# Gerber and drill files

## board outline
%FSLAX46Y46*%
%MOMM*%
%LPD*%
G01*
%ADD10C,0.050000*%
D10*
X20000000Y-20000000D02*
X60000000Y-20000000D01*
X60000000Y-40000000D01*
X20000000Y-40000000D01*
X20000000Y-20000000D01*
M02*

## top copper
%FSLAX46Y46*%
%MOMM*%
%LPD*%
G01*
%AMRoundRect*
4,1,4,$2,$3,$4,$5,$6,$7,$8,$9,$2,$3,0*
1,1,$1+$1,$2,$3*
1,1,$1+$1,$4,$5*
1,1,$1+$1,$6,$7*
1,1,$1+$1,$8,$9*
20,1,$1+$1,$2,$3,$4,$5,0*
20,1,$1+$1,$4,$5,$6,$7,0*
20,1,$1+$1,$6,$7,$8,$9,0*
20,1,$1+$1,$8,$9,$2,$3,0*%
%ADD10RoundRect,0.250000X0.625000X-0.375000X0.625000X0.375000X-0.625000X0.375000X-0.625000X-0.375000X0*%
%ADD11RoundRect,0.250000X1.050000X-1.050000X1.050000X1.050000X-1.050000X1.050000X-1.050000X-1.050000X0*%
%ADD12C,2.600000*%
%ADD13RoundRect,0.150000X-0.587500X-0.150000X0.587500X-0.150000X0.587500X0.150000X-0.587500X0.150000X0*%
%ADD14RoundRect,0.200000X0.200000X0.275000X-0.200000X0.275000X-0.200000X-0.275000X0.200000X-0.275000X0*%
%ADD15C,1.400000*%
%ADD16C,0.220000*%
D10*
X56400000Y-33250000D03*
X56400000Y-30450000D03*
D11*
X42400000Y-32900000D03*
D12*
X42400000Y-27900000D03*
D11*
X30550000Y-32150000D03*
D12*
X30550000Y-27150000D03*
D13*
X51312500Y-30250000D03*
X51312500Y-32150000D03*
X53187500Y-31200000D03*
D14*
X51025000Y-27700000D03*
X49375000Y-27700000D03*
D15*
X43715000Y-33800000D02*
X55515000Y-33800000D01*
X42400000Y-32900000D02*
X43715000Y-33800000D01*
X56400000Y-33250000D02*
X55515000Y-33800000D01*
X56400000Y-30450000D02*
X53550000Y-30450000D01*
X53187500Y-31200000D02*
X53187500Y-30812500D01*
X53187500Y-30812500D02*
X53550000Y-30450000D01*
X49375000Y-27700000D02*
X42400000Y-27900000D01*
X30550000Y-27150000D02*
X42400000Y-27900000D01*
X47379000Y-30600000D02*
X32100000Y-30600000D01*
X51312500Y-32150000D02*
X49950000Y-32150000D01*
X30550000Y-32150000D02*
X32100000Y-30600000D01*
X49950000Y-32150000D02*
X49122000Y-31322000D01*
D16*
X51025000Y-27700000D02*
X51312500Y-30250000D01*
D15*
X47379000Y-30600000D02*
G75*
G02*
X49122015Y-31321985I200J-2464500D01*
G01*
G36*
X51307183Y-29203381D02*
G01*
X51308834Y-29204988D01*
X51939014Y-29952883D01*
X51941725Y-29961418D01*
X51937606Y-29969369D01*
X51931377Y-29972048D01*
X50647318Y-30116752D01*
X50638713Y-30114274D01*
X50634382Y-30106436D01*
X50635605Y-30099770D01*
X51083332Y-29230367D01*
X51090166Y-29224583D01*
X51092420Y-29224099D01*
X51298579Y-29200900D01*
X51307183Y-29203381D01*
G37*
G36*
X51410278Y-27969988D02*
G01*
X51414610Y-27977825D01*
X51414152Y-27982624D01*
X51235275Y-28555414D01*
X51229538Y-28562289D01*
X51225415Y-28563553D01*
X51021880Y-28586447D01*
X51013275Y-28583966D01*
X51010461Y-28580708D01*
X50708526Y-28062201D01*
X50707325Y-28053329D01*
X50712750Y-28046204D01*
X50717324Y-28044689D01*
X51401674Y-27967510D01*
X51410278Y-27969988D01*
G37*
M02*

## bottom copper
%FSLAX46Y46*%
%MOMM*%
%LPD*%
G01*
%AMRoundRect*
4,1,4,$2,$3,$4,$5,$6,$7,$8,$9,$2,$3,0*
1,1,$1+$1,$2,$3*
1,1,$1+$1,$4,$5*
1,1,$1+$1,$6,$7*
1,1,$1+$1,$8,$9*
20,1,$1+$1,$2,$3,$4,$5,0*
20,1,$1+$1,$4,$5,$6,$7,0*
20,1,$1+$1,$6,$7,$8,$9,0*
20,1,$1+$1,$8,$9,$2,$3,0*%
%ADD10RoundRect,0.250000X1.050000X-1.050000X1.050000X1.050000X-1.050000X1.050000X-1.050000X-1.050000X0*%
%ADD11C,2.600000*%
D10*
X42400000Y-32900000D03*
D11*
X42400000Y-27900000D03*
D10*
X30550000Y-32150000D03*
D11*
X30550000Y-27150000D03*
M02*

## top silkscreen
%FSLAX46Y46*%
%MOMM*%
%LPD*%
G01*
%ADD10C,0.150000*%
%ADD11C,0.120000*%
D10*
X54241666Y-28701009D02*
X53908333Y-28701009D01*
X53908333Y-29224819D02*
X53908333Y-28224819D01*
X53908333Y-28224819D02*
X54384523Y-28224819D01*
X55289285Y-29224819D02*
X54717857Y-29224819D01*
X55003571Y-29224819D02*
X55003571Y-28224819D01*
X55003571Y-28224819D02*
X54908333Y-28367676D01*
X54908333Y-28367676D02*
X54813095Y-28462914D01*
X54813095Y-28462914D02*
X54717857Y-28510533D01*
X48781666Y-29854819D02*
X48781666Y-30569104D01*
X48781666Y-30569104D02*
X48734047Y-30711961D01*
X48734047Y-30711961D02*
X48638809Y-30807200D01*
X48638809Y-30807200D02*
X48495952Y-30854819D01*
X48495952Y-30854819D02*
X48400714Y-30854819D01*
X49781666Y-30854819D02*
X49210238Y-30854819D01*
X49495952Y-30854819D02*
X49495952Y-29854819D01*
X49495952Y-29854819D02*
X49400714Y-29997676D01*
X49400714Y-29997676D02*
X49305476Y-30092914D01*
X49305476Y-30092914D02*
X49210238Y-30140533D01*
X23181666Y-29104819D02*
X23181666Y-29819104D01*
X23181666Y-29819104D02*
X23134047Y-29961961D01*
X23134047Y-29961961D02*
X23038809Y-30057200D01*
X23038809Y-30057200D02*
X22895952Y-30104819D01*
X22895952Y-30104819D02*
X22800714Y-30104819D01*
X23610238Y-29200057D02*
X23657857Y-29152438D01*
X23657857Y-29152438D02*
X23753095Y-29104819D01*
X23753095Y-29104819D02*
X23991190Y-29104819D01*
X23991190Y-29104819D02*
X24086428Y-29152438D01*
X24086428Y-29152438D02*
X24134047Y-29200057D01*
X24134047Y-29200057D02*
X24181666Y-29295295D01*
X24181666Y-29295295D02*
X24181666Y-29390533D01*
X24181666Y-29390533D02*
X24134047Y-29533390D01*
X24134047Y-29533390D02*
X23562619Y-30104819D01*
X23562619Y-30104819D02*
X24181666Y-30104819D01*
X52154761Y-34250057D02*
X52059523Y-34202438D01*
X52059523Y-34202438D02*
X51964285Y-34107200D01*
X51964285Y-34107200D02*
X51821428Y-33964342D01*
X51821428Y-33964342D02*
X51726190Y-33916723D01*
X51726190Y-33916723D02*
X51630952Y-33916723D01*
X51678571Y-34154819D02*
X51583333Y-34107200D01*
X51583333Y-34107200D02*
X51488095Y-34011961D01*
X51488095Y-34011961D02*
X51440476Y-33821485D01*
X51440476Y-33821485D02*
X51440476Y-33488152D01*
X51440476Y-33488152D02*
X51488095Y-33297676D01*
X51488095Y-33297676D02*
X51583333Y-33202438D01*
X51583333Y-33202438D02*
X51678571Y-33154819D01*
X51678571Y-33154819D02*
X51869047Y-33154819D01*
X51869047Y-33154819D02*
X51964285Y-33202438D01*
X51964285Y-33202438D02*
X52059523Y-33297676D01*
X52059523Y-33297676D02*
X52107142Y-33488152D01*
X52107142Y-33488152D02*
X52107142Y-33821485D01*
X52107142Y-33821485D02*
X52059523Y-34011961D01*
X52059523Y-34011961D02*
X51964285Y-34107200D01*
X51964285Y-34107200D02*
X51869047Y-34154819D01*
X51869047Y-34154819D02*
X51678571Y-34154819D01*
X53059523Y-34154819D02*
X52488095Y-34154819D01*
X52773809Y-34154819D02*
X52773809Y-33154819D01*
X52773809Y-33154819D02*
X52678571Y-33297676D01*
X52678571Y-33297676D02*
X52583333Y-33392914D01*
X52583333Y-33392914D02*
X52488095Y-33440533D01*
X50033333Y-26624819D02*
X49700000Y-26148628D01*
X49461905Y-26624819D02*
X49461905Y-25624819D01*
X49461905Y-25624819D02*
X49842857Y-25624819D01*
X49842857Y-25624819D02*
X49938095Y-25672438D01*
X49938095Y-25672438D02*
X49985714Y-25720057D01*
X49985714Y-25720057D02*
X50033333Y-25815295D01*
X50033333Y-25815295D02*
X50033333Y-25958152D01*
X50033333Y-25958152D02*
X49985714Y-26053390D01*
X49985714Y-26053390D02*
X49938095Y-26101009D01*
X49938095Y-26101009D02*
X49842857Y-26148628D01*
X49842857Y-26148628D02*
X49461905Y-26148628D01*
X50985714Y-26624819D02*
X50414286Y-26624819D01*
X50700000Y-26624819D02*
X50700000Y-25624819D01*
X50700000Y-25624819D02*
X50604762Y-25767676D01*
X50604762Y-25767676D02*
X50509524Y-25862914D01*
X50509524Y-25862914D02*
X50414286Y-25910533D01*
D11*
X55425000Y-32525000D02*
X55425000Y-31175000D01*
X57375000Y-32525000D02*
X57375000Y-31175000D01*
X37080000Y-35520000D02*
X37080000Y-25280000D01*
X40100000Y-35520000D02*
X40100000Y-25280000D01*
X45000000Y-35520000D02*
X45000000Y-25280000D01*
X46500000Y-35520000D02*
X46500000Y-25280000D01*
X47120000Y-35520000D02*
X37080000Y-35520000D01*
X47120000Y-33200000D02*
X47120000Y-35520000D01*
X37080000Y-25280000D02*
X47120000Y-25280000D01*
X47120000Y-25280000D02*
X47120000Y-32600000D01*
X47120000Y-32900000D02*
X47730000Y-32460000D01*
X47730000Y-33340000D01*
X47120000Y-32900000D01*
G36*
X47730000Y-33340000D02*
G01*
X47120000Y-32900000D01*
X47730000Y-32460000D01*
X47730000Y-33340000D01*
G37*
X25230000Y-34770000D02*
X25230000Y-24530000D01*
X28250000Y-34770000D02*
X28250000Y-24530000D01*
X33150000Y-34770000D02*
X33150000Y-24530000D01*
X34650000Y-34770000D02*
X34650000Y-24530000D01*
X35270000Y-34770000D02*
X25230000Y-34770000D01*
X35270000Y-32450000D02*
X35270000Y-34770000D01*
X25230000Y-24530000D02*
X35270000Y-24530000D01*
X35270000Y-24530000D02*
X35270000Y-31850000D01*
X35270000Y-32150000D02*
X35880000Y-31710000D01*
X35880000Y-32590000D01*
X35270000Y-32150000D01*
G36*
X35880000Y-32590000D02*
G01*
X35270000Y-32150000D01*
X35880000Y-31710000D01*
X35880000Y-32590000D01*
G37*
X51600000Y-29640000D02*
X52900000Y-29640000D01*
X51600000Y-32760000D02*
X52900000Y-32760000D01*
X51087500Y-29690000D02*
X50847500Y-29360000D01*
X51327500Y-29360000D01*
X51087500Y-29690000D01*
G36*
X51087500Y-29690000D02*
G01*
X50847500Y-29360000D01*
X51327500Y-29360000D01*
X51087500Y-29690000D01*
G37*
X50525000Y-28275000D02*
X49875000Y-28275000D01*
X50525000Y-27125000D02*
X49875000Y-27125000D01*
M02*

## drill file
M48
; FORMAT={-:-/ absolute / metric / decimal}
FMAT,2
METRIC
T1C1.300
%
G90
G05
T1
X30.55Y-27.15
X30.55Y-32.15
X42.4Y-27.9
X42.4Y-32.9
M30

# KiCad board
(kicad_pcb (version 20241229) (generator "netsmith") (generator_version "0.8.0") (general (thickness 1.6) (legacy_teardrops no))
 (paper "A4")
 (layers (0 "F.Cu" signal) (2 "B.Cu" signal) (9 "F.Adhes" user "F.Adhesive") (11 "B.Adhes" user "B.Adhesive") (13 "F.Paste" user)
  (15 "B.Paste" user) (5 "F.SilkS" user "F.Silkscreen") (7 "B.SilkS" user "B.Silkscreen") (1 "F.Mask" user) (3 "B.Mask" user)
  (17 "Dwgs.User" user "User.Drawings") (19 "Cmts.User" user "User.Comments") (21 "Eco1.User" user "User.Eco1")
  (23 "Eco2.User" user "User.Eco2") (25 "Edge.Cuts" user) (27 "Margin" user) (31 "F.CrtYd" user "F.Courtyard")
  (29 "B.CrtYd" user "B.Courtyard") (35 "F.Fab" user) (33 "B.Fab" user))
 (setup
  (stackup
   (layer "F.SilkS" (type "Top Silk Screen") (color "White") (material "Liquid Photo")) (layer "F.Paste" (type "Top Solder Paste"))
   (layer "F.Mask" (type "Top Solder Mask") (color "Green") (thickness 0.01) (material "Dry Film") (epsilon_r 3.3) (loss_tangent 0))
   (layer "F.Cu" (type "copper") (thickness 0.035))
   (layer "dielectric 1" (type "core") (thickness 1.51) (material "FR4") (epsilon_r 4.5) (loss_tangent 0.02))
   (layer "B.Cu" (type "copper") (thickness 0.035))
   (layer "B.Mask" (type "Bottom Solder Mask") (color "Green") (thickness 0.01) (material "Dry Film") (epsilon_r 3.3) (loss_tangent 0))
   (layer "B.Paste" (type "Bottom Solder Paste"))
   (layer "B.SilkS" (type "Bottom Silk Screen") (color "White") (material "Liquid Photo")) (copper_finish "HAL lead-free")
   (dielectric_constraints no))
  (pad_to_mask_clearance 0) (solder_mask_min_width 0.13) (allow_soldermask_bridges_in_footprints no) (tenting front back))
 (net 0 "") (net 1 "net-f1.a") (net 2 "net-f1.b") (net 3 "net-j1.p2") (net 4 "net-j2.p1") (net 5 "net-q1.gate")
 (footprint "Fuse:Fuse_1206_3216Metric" (layer "F.Cu") (at 56.4 31.85 90)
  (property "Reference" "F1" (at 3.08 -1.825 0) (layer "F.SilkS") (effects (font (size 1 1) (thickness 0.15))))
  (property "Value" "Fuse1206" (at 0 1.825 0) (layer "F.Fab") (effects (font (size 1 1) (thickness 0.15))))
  (pad "1" smd roundrect (at -1.4 0 90) (size 1.25 1.75) (layers "F.Cu" "F.Mask" "F.Paste") (roundrect_rratio 0.2) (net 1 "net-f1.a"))
  (pad "2" smd roundrect (at 1.4 0 90) (size 1.25 1.75) (layers "F.Cu" "F.Mask" "F.Paste") (roundrect_rratio 0.2) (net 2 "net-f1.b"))
  (fp_line (start -0.675 -0.975) (end 0.675 -0.975) (stroke (width 0.12) (type solid)) (layer "F.SilkS"))
  (fp_line (start -0.675 0.975) (end 0.675 0.975) (stroke (width 0.12) (type solid)) (layer "F.SilkS")))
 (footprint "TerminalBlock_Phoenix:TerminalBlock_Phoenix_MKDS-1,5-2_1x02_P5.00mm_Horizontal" (layer "F.Cu") (at 42.4 32.9 90)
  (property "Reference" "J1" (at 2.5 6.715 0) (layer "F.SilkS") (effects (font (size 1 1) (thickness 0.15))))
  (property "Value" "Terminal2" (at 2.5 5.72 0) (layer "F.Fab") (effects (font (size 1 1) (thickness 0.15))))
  (fp_line (start -2.62 -5.32) (end 7.62 -5.32) (stroke (width 0.12) (type solid)) (layer "F.SilkS"))
  (fp_line (start -2.62 -2.3) (end 7.62 -2.3) (stroke (width 0.12) (type solid)) (layer "F.SilkS"))
  (fp_line (start -2.62 2.6) (end 7.62 2.6) (stroke (width 0.12) (type solid)) (layer "F.SilkS"))
  (fp_line (start -2.62 4.1) (end 7.62 4.1) (stroke (width 0.12) (type solid)) (layer "F.SilkS"))
  (fp_line (start -2.62 4.72) (end -2.62 -5.32) (stroke (width 0.12) (type solid)) (layer "F.SilkS"))
  (fp_line (start -0.3 4.72) (end -2.62 4.72) (stroke (width 0.12) (type solid)) (layer "F.SilkS"))
  (fp_line (start 7.62 -5.32) (end 7.62 4.72) (stroke (width 0.12) (type solid)) (layer "F.SilkS"))
  (fp_line (start 7.62 4.72) (end 0.3 4.72) (stroke (width 0.12) (type solid)) (layer "F.SilkS"))
  (fp_poly (pts (xy 0 4.72) (xy 0.44 5.33) (xy -0.44 5.33)) (stroke (width 0.12) (type solid)) (fill yes) (layer "F.SilkS"))
  (pad "1" thru_hole roundrect (at 0 0 90) (size 2.6 2.6) (drill 1.3) (layers "*.Cu" "*.Mask") (remove_unused_layers no)
   (roundrect_rratio 0.096154) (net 1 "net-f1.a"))
  (pad "2" thru_hole circle (at 5 0 90) (size 2.6 2.6) (drill 1.3) (layers "*.Cu" "*.Mask") (remove_unused_layers no) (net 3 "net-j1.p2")))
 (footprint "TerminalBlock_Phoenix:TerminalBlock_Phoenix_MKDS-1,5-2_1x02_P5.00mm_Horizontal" (layer "F.Cu") (at 30.55 32.15 90)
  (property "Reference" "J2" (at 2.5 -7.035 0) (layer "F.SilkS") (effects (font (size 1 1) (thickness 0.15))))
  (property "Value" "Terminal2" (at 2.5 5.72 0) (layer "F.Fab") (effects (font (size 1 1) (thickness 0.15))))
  (fp_line (start -2.62 -5.32) (end 7.62 -5.32) (stroke (width 0.12) (type solid)) (layer "F.SilkS"))
  (fp_line (start -2.62 -2.3) (end 7.62 -2.3) (stroke (width 0.12) (type solid)) (layer "F.SilkS"))
  (fp_line (start -2.62 2.6) (end 7.62 2.6) (stroke (width 0.12) (type solid)) (layer "F.SilkS"))
  (fp_line (start -2.62 4.1) (end 7.62 4.1) (stroke (width 0.12) (type solid)) (layer "F.SilkS"))
  (fp_line (start -2.62 4.72) (end -2.62 -5.32) (stroke (width 0.12) (type solid)) (layer "F.SilkS"))
  (fp_line (start -0.3 4.72) (end -2.62 4.72) (stroke (width 0.12) (type solid)) (layer "F.SilkS"))
  (fp_line (start 7.62 -5.32) (end 7.62 4.72) (stroke (width 0.12) (type solid)) (layer "F.SilkS"))
  (fp_line (start 7.62 4.72) (end 0.3 4.72) (stroke (width 0.12) (type solid)) (layer "F.SilkS"))
  (fp_poly (pts (xy 0 4.72) (xy 0.44 5.33) (xy -0.44 5.33)) (stroke (width 0.12) (type solid)) (fill yes) (layer "F.SilkS"))
  (pad "1" thru_hole roundrect (at 0 0 90) (size 2.6 2.6) (drill 1.3) (layers "*.Cu" "*.Mask") (remove_unused_layers no)
   (roundrect_rratio 0.096154) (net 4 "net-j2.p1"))
  (pad "2" thru_hole circle (at 5 0 90) (size 2.6 2.6) (drill 1.3) (layers "*.Cu" "*.Mask") (remove_unused_layers no) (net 3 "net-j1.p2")))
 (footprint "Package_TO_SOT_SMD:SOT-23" (layer "F.Cu") (at 52.25 31.2)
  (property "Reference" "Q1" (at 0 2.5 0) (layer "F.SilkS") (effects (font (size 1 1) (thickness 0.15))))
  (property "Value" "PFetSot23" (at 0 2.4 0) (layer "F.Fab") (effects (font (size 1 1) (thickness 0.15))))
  (pad "1" smd roundrect (at -0.9375 -0.95) (size 1.475 0.6) (layers "F.Cu" "F.Mask" "F.Paste") (roundrect_rratio 0.25)
   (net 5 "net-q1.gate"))
  (pad "2" smd roundrect (at -0.9375 0.95) (size 1.475 0.6) (layers "F.Cu" "F.Mask" "F.Paste") (roundrect_rratio 0.25) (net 4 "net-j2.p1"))
  (pad "3" smd roundrect (at 0.9375 0) (size 1.475 0.6) (layers "F.Cu" "F.Mask" "F.Paste") (roundrect_rratio 0.25) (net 2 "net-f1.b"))
  (fp_line (start -0.65 -1.56) (end 0.65 -1.56) (stroke (width 0.12) (type solid)) (layer "F.SilkS"))
  (fp_line (start -0.65 1.56) (end 0.65 1.56) (stroke (width 0.12) (type solid)) (layer "F.SilkS"))
  (fp_poly (pts (xy -1.1625 -1.51) (xy -1.4025 -1.84) (xy -0.9225 -1.84)) (stroke (width 0.12) (type solid)) (fill solid) (layer "F.SilkS")))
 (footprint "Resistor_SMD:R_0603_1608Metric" (layer "F.Cu") (at 50.2 27.7 180)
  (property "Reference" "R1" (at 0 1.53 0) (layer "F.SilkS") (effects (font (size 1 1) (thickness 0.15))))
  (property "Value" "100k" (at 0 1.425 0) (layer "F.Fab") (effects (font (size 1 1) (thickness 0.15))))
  (pad "1" smd roundrect (at -0.825 0 180) (size 0.8 0.95) (layers "F.Cu" "F.Mask" "F.Paste") (roundrect_rratio 0.25) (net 5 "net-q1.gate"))
  (pad "2" smd roundrect (at 0.825 0 180) (size 0.8 0.95) (layers "F.Cu" "F.Mask" "F.Paste") (roundrect_rratio 0.25) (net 3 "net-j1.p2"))
  (fp_line (start -0.325 -0.575) (end 0.325 -0.575) (stroke (width 0.12) (type solid)) (layer "F.SilkS"))
  (fp_line (start -0.325 0.575) (end 0.325 0.575) (stroke (width 0.12) (type solid)) (layer "F.SilkS")))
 (segment (start 43.715 33.8) (end 55.515 33.8) (width 1.4) (layer "F.Cu") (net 1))
 (segment (start 42.4 32.9) (end 43.715 33.8) (width 1.4) (layer "F.Cu") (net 1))
 (segment (start 56.4 33.25) (end 55.515 33.8) (width 1.4) (layer "F.Cu") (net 1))
 (segment (start 56.4 30.45) (end 53.55 30.45) (width 1.4) (layer "F.Cu") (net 2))
 (segment (start 53.1875 31.2) (end 53.1875 30.8125) (width 1.4) (layer "F.Cu") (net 2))
 (segment (start 53.1875 30.8125) (end 53.55 30.45) (width 1.4) (layer "F.Cu") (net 2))
 (segment (start 49.375 27.7) (end 42.4 27.9) (width 1.4) (layer "F.Cu") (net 3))
 (segment (start 30.55 27.15) (end 42.4 27.9) (width 1.4) (layer "F.Cu") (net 3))
 (segment (start 47.379 30.6) (end 32.1 30.6) (width 1.4) (layer "F.Cu") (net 4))
 (segment (start 51.3125 32.15) (end 49.95 32.15) (width 1.4) (layer "F.Cu") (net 4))
 (segment (start 30.55 32.15) (end 32.1 30.6) (width 1.4) (layer "F.Cu") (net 4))
 (segment (start 49.95 32.15) (end 49.122 31.322) (width 1.4) (layer "F.Cu") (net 4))
 (segment (start 51.025 27.7) (end 51.3125 30.25) (width 0.22) (layer "F.Cu") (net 5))
 (arc (start 47.379 30.6) (mid 48.3223 30.7876) (end 49.122 31.322) (width 1.4) (layer "F.Cu") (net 4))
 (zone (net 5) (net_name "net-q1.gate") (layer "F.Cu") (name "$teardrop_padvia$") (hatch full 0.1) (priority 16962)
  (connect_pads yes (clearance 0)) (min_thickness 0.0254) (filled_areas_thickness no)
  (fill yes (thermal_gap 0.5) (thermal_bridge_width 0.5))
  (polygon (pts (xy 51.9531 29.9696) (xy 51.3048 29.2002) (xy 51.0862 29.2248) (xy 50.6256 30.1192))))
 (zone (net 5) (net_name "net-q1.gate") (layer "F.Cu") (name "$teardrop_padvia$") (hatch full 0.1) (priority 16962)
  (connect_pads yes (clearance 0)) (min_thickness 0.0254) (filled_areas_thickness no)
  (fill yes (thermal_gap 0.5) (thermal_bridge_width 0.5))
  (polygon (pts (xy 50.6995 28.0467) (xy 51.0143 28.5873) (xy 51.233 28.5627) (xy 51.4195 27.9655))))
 (gr_rect (start 20 20) (end 60 40) (stroke (width 0.05) (type default)) (fill no) (layer "Edge.Cuts")))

